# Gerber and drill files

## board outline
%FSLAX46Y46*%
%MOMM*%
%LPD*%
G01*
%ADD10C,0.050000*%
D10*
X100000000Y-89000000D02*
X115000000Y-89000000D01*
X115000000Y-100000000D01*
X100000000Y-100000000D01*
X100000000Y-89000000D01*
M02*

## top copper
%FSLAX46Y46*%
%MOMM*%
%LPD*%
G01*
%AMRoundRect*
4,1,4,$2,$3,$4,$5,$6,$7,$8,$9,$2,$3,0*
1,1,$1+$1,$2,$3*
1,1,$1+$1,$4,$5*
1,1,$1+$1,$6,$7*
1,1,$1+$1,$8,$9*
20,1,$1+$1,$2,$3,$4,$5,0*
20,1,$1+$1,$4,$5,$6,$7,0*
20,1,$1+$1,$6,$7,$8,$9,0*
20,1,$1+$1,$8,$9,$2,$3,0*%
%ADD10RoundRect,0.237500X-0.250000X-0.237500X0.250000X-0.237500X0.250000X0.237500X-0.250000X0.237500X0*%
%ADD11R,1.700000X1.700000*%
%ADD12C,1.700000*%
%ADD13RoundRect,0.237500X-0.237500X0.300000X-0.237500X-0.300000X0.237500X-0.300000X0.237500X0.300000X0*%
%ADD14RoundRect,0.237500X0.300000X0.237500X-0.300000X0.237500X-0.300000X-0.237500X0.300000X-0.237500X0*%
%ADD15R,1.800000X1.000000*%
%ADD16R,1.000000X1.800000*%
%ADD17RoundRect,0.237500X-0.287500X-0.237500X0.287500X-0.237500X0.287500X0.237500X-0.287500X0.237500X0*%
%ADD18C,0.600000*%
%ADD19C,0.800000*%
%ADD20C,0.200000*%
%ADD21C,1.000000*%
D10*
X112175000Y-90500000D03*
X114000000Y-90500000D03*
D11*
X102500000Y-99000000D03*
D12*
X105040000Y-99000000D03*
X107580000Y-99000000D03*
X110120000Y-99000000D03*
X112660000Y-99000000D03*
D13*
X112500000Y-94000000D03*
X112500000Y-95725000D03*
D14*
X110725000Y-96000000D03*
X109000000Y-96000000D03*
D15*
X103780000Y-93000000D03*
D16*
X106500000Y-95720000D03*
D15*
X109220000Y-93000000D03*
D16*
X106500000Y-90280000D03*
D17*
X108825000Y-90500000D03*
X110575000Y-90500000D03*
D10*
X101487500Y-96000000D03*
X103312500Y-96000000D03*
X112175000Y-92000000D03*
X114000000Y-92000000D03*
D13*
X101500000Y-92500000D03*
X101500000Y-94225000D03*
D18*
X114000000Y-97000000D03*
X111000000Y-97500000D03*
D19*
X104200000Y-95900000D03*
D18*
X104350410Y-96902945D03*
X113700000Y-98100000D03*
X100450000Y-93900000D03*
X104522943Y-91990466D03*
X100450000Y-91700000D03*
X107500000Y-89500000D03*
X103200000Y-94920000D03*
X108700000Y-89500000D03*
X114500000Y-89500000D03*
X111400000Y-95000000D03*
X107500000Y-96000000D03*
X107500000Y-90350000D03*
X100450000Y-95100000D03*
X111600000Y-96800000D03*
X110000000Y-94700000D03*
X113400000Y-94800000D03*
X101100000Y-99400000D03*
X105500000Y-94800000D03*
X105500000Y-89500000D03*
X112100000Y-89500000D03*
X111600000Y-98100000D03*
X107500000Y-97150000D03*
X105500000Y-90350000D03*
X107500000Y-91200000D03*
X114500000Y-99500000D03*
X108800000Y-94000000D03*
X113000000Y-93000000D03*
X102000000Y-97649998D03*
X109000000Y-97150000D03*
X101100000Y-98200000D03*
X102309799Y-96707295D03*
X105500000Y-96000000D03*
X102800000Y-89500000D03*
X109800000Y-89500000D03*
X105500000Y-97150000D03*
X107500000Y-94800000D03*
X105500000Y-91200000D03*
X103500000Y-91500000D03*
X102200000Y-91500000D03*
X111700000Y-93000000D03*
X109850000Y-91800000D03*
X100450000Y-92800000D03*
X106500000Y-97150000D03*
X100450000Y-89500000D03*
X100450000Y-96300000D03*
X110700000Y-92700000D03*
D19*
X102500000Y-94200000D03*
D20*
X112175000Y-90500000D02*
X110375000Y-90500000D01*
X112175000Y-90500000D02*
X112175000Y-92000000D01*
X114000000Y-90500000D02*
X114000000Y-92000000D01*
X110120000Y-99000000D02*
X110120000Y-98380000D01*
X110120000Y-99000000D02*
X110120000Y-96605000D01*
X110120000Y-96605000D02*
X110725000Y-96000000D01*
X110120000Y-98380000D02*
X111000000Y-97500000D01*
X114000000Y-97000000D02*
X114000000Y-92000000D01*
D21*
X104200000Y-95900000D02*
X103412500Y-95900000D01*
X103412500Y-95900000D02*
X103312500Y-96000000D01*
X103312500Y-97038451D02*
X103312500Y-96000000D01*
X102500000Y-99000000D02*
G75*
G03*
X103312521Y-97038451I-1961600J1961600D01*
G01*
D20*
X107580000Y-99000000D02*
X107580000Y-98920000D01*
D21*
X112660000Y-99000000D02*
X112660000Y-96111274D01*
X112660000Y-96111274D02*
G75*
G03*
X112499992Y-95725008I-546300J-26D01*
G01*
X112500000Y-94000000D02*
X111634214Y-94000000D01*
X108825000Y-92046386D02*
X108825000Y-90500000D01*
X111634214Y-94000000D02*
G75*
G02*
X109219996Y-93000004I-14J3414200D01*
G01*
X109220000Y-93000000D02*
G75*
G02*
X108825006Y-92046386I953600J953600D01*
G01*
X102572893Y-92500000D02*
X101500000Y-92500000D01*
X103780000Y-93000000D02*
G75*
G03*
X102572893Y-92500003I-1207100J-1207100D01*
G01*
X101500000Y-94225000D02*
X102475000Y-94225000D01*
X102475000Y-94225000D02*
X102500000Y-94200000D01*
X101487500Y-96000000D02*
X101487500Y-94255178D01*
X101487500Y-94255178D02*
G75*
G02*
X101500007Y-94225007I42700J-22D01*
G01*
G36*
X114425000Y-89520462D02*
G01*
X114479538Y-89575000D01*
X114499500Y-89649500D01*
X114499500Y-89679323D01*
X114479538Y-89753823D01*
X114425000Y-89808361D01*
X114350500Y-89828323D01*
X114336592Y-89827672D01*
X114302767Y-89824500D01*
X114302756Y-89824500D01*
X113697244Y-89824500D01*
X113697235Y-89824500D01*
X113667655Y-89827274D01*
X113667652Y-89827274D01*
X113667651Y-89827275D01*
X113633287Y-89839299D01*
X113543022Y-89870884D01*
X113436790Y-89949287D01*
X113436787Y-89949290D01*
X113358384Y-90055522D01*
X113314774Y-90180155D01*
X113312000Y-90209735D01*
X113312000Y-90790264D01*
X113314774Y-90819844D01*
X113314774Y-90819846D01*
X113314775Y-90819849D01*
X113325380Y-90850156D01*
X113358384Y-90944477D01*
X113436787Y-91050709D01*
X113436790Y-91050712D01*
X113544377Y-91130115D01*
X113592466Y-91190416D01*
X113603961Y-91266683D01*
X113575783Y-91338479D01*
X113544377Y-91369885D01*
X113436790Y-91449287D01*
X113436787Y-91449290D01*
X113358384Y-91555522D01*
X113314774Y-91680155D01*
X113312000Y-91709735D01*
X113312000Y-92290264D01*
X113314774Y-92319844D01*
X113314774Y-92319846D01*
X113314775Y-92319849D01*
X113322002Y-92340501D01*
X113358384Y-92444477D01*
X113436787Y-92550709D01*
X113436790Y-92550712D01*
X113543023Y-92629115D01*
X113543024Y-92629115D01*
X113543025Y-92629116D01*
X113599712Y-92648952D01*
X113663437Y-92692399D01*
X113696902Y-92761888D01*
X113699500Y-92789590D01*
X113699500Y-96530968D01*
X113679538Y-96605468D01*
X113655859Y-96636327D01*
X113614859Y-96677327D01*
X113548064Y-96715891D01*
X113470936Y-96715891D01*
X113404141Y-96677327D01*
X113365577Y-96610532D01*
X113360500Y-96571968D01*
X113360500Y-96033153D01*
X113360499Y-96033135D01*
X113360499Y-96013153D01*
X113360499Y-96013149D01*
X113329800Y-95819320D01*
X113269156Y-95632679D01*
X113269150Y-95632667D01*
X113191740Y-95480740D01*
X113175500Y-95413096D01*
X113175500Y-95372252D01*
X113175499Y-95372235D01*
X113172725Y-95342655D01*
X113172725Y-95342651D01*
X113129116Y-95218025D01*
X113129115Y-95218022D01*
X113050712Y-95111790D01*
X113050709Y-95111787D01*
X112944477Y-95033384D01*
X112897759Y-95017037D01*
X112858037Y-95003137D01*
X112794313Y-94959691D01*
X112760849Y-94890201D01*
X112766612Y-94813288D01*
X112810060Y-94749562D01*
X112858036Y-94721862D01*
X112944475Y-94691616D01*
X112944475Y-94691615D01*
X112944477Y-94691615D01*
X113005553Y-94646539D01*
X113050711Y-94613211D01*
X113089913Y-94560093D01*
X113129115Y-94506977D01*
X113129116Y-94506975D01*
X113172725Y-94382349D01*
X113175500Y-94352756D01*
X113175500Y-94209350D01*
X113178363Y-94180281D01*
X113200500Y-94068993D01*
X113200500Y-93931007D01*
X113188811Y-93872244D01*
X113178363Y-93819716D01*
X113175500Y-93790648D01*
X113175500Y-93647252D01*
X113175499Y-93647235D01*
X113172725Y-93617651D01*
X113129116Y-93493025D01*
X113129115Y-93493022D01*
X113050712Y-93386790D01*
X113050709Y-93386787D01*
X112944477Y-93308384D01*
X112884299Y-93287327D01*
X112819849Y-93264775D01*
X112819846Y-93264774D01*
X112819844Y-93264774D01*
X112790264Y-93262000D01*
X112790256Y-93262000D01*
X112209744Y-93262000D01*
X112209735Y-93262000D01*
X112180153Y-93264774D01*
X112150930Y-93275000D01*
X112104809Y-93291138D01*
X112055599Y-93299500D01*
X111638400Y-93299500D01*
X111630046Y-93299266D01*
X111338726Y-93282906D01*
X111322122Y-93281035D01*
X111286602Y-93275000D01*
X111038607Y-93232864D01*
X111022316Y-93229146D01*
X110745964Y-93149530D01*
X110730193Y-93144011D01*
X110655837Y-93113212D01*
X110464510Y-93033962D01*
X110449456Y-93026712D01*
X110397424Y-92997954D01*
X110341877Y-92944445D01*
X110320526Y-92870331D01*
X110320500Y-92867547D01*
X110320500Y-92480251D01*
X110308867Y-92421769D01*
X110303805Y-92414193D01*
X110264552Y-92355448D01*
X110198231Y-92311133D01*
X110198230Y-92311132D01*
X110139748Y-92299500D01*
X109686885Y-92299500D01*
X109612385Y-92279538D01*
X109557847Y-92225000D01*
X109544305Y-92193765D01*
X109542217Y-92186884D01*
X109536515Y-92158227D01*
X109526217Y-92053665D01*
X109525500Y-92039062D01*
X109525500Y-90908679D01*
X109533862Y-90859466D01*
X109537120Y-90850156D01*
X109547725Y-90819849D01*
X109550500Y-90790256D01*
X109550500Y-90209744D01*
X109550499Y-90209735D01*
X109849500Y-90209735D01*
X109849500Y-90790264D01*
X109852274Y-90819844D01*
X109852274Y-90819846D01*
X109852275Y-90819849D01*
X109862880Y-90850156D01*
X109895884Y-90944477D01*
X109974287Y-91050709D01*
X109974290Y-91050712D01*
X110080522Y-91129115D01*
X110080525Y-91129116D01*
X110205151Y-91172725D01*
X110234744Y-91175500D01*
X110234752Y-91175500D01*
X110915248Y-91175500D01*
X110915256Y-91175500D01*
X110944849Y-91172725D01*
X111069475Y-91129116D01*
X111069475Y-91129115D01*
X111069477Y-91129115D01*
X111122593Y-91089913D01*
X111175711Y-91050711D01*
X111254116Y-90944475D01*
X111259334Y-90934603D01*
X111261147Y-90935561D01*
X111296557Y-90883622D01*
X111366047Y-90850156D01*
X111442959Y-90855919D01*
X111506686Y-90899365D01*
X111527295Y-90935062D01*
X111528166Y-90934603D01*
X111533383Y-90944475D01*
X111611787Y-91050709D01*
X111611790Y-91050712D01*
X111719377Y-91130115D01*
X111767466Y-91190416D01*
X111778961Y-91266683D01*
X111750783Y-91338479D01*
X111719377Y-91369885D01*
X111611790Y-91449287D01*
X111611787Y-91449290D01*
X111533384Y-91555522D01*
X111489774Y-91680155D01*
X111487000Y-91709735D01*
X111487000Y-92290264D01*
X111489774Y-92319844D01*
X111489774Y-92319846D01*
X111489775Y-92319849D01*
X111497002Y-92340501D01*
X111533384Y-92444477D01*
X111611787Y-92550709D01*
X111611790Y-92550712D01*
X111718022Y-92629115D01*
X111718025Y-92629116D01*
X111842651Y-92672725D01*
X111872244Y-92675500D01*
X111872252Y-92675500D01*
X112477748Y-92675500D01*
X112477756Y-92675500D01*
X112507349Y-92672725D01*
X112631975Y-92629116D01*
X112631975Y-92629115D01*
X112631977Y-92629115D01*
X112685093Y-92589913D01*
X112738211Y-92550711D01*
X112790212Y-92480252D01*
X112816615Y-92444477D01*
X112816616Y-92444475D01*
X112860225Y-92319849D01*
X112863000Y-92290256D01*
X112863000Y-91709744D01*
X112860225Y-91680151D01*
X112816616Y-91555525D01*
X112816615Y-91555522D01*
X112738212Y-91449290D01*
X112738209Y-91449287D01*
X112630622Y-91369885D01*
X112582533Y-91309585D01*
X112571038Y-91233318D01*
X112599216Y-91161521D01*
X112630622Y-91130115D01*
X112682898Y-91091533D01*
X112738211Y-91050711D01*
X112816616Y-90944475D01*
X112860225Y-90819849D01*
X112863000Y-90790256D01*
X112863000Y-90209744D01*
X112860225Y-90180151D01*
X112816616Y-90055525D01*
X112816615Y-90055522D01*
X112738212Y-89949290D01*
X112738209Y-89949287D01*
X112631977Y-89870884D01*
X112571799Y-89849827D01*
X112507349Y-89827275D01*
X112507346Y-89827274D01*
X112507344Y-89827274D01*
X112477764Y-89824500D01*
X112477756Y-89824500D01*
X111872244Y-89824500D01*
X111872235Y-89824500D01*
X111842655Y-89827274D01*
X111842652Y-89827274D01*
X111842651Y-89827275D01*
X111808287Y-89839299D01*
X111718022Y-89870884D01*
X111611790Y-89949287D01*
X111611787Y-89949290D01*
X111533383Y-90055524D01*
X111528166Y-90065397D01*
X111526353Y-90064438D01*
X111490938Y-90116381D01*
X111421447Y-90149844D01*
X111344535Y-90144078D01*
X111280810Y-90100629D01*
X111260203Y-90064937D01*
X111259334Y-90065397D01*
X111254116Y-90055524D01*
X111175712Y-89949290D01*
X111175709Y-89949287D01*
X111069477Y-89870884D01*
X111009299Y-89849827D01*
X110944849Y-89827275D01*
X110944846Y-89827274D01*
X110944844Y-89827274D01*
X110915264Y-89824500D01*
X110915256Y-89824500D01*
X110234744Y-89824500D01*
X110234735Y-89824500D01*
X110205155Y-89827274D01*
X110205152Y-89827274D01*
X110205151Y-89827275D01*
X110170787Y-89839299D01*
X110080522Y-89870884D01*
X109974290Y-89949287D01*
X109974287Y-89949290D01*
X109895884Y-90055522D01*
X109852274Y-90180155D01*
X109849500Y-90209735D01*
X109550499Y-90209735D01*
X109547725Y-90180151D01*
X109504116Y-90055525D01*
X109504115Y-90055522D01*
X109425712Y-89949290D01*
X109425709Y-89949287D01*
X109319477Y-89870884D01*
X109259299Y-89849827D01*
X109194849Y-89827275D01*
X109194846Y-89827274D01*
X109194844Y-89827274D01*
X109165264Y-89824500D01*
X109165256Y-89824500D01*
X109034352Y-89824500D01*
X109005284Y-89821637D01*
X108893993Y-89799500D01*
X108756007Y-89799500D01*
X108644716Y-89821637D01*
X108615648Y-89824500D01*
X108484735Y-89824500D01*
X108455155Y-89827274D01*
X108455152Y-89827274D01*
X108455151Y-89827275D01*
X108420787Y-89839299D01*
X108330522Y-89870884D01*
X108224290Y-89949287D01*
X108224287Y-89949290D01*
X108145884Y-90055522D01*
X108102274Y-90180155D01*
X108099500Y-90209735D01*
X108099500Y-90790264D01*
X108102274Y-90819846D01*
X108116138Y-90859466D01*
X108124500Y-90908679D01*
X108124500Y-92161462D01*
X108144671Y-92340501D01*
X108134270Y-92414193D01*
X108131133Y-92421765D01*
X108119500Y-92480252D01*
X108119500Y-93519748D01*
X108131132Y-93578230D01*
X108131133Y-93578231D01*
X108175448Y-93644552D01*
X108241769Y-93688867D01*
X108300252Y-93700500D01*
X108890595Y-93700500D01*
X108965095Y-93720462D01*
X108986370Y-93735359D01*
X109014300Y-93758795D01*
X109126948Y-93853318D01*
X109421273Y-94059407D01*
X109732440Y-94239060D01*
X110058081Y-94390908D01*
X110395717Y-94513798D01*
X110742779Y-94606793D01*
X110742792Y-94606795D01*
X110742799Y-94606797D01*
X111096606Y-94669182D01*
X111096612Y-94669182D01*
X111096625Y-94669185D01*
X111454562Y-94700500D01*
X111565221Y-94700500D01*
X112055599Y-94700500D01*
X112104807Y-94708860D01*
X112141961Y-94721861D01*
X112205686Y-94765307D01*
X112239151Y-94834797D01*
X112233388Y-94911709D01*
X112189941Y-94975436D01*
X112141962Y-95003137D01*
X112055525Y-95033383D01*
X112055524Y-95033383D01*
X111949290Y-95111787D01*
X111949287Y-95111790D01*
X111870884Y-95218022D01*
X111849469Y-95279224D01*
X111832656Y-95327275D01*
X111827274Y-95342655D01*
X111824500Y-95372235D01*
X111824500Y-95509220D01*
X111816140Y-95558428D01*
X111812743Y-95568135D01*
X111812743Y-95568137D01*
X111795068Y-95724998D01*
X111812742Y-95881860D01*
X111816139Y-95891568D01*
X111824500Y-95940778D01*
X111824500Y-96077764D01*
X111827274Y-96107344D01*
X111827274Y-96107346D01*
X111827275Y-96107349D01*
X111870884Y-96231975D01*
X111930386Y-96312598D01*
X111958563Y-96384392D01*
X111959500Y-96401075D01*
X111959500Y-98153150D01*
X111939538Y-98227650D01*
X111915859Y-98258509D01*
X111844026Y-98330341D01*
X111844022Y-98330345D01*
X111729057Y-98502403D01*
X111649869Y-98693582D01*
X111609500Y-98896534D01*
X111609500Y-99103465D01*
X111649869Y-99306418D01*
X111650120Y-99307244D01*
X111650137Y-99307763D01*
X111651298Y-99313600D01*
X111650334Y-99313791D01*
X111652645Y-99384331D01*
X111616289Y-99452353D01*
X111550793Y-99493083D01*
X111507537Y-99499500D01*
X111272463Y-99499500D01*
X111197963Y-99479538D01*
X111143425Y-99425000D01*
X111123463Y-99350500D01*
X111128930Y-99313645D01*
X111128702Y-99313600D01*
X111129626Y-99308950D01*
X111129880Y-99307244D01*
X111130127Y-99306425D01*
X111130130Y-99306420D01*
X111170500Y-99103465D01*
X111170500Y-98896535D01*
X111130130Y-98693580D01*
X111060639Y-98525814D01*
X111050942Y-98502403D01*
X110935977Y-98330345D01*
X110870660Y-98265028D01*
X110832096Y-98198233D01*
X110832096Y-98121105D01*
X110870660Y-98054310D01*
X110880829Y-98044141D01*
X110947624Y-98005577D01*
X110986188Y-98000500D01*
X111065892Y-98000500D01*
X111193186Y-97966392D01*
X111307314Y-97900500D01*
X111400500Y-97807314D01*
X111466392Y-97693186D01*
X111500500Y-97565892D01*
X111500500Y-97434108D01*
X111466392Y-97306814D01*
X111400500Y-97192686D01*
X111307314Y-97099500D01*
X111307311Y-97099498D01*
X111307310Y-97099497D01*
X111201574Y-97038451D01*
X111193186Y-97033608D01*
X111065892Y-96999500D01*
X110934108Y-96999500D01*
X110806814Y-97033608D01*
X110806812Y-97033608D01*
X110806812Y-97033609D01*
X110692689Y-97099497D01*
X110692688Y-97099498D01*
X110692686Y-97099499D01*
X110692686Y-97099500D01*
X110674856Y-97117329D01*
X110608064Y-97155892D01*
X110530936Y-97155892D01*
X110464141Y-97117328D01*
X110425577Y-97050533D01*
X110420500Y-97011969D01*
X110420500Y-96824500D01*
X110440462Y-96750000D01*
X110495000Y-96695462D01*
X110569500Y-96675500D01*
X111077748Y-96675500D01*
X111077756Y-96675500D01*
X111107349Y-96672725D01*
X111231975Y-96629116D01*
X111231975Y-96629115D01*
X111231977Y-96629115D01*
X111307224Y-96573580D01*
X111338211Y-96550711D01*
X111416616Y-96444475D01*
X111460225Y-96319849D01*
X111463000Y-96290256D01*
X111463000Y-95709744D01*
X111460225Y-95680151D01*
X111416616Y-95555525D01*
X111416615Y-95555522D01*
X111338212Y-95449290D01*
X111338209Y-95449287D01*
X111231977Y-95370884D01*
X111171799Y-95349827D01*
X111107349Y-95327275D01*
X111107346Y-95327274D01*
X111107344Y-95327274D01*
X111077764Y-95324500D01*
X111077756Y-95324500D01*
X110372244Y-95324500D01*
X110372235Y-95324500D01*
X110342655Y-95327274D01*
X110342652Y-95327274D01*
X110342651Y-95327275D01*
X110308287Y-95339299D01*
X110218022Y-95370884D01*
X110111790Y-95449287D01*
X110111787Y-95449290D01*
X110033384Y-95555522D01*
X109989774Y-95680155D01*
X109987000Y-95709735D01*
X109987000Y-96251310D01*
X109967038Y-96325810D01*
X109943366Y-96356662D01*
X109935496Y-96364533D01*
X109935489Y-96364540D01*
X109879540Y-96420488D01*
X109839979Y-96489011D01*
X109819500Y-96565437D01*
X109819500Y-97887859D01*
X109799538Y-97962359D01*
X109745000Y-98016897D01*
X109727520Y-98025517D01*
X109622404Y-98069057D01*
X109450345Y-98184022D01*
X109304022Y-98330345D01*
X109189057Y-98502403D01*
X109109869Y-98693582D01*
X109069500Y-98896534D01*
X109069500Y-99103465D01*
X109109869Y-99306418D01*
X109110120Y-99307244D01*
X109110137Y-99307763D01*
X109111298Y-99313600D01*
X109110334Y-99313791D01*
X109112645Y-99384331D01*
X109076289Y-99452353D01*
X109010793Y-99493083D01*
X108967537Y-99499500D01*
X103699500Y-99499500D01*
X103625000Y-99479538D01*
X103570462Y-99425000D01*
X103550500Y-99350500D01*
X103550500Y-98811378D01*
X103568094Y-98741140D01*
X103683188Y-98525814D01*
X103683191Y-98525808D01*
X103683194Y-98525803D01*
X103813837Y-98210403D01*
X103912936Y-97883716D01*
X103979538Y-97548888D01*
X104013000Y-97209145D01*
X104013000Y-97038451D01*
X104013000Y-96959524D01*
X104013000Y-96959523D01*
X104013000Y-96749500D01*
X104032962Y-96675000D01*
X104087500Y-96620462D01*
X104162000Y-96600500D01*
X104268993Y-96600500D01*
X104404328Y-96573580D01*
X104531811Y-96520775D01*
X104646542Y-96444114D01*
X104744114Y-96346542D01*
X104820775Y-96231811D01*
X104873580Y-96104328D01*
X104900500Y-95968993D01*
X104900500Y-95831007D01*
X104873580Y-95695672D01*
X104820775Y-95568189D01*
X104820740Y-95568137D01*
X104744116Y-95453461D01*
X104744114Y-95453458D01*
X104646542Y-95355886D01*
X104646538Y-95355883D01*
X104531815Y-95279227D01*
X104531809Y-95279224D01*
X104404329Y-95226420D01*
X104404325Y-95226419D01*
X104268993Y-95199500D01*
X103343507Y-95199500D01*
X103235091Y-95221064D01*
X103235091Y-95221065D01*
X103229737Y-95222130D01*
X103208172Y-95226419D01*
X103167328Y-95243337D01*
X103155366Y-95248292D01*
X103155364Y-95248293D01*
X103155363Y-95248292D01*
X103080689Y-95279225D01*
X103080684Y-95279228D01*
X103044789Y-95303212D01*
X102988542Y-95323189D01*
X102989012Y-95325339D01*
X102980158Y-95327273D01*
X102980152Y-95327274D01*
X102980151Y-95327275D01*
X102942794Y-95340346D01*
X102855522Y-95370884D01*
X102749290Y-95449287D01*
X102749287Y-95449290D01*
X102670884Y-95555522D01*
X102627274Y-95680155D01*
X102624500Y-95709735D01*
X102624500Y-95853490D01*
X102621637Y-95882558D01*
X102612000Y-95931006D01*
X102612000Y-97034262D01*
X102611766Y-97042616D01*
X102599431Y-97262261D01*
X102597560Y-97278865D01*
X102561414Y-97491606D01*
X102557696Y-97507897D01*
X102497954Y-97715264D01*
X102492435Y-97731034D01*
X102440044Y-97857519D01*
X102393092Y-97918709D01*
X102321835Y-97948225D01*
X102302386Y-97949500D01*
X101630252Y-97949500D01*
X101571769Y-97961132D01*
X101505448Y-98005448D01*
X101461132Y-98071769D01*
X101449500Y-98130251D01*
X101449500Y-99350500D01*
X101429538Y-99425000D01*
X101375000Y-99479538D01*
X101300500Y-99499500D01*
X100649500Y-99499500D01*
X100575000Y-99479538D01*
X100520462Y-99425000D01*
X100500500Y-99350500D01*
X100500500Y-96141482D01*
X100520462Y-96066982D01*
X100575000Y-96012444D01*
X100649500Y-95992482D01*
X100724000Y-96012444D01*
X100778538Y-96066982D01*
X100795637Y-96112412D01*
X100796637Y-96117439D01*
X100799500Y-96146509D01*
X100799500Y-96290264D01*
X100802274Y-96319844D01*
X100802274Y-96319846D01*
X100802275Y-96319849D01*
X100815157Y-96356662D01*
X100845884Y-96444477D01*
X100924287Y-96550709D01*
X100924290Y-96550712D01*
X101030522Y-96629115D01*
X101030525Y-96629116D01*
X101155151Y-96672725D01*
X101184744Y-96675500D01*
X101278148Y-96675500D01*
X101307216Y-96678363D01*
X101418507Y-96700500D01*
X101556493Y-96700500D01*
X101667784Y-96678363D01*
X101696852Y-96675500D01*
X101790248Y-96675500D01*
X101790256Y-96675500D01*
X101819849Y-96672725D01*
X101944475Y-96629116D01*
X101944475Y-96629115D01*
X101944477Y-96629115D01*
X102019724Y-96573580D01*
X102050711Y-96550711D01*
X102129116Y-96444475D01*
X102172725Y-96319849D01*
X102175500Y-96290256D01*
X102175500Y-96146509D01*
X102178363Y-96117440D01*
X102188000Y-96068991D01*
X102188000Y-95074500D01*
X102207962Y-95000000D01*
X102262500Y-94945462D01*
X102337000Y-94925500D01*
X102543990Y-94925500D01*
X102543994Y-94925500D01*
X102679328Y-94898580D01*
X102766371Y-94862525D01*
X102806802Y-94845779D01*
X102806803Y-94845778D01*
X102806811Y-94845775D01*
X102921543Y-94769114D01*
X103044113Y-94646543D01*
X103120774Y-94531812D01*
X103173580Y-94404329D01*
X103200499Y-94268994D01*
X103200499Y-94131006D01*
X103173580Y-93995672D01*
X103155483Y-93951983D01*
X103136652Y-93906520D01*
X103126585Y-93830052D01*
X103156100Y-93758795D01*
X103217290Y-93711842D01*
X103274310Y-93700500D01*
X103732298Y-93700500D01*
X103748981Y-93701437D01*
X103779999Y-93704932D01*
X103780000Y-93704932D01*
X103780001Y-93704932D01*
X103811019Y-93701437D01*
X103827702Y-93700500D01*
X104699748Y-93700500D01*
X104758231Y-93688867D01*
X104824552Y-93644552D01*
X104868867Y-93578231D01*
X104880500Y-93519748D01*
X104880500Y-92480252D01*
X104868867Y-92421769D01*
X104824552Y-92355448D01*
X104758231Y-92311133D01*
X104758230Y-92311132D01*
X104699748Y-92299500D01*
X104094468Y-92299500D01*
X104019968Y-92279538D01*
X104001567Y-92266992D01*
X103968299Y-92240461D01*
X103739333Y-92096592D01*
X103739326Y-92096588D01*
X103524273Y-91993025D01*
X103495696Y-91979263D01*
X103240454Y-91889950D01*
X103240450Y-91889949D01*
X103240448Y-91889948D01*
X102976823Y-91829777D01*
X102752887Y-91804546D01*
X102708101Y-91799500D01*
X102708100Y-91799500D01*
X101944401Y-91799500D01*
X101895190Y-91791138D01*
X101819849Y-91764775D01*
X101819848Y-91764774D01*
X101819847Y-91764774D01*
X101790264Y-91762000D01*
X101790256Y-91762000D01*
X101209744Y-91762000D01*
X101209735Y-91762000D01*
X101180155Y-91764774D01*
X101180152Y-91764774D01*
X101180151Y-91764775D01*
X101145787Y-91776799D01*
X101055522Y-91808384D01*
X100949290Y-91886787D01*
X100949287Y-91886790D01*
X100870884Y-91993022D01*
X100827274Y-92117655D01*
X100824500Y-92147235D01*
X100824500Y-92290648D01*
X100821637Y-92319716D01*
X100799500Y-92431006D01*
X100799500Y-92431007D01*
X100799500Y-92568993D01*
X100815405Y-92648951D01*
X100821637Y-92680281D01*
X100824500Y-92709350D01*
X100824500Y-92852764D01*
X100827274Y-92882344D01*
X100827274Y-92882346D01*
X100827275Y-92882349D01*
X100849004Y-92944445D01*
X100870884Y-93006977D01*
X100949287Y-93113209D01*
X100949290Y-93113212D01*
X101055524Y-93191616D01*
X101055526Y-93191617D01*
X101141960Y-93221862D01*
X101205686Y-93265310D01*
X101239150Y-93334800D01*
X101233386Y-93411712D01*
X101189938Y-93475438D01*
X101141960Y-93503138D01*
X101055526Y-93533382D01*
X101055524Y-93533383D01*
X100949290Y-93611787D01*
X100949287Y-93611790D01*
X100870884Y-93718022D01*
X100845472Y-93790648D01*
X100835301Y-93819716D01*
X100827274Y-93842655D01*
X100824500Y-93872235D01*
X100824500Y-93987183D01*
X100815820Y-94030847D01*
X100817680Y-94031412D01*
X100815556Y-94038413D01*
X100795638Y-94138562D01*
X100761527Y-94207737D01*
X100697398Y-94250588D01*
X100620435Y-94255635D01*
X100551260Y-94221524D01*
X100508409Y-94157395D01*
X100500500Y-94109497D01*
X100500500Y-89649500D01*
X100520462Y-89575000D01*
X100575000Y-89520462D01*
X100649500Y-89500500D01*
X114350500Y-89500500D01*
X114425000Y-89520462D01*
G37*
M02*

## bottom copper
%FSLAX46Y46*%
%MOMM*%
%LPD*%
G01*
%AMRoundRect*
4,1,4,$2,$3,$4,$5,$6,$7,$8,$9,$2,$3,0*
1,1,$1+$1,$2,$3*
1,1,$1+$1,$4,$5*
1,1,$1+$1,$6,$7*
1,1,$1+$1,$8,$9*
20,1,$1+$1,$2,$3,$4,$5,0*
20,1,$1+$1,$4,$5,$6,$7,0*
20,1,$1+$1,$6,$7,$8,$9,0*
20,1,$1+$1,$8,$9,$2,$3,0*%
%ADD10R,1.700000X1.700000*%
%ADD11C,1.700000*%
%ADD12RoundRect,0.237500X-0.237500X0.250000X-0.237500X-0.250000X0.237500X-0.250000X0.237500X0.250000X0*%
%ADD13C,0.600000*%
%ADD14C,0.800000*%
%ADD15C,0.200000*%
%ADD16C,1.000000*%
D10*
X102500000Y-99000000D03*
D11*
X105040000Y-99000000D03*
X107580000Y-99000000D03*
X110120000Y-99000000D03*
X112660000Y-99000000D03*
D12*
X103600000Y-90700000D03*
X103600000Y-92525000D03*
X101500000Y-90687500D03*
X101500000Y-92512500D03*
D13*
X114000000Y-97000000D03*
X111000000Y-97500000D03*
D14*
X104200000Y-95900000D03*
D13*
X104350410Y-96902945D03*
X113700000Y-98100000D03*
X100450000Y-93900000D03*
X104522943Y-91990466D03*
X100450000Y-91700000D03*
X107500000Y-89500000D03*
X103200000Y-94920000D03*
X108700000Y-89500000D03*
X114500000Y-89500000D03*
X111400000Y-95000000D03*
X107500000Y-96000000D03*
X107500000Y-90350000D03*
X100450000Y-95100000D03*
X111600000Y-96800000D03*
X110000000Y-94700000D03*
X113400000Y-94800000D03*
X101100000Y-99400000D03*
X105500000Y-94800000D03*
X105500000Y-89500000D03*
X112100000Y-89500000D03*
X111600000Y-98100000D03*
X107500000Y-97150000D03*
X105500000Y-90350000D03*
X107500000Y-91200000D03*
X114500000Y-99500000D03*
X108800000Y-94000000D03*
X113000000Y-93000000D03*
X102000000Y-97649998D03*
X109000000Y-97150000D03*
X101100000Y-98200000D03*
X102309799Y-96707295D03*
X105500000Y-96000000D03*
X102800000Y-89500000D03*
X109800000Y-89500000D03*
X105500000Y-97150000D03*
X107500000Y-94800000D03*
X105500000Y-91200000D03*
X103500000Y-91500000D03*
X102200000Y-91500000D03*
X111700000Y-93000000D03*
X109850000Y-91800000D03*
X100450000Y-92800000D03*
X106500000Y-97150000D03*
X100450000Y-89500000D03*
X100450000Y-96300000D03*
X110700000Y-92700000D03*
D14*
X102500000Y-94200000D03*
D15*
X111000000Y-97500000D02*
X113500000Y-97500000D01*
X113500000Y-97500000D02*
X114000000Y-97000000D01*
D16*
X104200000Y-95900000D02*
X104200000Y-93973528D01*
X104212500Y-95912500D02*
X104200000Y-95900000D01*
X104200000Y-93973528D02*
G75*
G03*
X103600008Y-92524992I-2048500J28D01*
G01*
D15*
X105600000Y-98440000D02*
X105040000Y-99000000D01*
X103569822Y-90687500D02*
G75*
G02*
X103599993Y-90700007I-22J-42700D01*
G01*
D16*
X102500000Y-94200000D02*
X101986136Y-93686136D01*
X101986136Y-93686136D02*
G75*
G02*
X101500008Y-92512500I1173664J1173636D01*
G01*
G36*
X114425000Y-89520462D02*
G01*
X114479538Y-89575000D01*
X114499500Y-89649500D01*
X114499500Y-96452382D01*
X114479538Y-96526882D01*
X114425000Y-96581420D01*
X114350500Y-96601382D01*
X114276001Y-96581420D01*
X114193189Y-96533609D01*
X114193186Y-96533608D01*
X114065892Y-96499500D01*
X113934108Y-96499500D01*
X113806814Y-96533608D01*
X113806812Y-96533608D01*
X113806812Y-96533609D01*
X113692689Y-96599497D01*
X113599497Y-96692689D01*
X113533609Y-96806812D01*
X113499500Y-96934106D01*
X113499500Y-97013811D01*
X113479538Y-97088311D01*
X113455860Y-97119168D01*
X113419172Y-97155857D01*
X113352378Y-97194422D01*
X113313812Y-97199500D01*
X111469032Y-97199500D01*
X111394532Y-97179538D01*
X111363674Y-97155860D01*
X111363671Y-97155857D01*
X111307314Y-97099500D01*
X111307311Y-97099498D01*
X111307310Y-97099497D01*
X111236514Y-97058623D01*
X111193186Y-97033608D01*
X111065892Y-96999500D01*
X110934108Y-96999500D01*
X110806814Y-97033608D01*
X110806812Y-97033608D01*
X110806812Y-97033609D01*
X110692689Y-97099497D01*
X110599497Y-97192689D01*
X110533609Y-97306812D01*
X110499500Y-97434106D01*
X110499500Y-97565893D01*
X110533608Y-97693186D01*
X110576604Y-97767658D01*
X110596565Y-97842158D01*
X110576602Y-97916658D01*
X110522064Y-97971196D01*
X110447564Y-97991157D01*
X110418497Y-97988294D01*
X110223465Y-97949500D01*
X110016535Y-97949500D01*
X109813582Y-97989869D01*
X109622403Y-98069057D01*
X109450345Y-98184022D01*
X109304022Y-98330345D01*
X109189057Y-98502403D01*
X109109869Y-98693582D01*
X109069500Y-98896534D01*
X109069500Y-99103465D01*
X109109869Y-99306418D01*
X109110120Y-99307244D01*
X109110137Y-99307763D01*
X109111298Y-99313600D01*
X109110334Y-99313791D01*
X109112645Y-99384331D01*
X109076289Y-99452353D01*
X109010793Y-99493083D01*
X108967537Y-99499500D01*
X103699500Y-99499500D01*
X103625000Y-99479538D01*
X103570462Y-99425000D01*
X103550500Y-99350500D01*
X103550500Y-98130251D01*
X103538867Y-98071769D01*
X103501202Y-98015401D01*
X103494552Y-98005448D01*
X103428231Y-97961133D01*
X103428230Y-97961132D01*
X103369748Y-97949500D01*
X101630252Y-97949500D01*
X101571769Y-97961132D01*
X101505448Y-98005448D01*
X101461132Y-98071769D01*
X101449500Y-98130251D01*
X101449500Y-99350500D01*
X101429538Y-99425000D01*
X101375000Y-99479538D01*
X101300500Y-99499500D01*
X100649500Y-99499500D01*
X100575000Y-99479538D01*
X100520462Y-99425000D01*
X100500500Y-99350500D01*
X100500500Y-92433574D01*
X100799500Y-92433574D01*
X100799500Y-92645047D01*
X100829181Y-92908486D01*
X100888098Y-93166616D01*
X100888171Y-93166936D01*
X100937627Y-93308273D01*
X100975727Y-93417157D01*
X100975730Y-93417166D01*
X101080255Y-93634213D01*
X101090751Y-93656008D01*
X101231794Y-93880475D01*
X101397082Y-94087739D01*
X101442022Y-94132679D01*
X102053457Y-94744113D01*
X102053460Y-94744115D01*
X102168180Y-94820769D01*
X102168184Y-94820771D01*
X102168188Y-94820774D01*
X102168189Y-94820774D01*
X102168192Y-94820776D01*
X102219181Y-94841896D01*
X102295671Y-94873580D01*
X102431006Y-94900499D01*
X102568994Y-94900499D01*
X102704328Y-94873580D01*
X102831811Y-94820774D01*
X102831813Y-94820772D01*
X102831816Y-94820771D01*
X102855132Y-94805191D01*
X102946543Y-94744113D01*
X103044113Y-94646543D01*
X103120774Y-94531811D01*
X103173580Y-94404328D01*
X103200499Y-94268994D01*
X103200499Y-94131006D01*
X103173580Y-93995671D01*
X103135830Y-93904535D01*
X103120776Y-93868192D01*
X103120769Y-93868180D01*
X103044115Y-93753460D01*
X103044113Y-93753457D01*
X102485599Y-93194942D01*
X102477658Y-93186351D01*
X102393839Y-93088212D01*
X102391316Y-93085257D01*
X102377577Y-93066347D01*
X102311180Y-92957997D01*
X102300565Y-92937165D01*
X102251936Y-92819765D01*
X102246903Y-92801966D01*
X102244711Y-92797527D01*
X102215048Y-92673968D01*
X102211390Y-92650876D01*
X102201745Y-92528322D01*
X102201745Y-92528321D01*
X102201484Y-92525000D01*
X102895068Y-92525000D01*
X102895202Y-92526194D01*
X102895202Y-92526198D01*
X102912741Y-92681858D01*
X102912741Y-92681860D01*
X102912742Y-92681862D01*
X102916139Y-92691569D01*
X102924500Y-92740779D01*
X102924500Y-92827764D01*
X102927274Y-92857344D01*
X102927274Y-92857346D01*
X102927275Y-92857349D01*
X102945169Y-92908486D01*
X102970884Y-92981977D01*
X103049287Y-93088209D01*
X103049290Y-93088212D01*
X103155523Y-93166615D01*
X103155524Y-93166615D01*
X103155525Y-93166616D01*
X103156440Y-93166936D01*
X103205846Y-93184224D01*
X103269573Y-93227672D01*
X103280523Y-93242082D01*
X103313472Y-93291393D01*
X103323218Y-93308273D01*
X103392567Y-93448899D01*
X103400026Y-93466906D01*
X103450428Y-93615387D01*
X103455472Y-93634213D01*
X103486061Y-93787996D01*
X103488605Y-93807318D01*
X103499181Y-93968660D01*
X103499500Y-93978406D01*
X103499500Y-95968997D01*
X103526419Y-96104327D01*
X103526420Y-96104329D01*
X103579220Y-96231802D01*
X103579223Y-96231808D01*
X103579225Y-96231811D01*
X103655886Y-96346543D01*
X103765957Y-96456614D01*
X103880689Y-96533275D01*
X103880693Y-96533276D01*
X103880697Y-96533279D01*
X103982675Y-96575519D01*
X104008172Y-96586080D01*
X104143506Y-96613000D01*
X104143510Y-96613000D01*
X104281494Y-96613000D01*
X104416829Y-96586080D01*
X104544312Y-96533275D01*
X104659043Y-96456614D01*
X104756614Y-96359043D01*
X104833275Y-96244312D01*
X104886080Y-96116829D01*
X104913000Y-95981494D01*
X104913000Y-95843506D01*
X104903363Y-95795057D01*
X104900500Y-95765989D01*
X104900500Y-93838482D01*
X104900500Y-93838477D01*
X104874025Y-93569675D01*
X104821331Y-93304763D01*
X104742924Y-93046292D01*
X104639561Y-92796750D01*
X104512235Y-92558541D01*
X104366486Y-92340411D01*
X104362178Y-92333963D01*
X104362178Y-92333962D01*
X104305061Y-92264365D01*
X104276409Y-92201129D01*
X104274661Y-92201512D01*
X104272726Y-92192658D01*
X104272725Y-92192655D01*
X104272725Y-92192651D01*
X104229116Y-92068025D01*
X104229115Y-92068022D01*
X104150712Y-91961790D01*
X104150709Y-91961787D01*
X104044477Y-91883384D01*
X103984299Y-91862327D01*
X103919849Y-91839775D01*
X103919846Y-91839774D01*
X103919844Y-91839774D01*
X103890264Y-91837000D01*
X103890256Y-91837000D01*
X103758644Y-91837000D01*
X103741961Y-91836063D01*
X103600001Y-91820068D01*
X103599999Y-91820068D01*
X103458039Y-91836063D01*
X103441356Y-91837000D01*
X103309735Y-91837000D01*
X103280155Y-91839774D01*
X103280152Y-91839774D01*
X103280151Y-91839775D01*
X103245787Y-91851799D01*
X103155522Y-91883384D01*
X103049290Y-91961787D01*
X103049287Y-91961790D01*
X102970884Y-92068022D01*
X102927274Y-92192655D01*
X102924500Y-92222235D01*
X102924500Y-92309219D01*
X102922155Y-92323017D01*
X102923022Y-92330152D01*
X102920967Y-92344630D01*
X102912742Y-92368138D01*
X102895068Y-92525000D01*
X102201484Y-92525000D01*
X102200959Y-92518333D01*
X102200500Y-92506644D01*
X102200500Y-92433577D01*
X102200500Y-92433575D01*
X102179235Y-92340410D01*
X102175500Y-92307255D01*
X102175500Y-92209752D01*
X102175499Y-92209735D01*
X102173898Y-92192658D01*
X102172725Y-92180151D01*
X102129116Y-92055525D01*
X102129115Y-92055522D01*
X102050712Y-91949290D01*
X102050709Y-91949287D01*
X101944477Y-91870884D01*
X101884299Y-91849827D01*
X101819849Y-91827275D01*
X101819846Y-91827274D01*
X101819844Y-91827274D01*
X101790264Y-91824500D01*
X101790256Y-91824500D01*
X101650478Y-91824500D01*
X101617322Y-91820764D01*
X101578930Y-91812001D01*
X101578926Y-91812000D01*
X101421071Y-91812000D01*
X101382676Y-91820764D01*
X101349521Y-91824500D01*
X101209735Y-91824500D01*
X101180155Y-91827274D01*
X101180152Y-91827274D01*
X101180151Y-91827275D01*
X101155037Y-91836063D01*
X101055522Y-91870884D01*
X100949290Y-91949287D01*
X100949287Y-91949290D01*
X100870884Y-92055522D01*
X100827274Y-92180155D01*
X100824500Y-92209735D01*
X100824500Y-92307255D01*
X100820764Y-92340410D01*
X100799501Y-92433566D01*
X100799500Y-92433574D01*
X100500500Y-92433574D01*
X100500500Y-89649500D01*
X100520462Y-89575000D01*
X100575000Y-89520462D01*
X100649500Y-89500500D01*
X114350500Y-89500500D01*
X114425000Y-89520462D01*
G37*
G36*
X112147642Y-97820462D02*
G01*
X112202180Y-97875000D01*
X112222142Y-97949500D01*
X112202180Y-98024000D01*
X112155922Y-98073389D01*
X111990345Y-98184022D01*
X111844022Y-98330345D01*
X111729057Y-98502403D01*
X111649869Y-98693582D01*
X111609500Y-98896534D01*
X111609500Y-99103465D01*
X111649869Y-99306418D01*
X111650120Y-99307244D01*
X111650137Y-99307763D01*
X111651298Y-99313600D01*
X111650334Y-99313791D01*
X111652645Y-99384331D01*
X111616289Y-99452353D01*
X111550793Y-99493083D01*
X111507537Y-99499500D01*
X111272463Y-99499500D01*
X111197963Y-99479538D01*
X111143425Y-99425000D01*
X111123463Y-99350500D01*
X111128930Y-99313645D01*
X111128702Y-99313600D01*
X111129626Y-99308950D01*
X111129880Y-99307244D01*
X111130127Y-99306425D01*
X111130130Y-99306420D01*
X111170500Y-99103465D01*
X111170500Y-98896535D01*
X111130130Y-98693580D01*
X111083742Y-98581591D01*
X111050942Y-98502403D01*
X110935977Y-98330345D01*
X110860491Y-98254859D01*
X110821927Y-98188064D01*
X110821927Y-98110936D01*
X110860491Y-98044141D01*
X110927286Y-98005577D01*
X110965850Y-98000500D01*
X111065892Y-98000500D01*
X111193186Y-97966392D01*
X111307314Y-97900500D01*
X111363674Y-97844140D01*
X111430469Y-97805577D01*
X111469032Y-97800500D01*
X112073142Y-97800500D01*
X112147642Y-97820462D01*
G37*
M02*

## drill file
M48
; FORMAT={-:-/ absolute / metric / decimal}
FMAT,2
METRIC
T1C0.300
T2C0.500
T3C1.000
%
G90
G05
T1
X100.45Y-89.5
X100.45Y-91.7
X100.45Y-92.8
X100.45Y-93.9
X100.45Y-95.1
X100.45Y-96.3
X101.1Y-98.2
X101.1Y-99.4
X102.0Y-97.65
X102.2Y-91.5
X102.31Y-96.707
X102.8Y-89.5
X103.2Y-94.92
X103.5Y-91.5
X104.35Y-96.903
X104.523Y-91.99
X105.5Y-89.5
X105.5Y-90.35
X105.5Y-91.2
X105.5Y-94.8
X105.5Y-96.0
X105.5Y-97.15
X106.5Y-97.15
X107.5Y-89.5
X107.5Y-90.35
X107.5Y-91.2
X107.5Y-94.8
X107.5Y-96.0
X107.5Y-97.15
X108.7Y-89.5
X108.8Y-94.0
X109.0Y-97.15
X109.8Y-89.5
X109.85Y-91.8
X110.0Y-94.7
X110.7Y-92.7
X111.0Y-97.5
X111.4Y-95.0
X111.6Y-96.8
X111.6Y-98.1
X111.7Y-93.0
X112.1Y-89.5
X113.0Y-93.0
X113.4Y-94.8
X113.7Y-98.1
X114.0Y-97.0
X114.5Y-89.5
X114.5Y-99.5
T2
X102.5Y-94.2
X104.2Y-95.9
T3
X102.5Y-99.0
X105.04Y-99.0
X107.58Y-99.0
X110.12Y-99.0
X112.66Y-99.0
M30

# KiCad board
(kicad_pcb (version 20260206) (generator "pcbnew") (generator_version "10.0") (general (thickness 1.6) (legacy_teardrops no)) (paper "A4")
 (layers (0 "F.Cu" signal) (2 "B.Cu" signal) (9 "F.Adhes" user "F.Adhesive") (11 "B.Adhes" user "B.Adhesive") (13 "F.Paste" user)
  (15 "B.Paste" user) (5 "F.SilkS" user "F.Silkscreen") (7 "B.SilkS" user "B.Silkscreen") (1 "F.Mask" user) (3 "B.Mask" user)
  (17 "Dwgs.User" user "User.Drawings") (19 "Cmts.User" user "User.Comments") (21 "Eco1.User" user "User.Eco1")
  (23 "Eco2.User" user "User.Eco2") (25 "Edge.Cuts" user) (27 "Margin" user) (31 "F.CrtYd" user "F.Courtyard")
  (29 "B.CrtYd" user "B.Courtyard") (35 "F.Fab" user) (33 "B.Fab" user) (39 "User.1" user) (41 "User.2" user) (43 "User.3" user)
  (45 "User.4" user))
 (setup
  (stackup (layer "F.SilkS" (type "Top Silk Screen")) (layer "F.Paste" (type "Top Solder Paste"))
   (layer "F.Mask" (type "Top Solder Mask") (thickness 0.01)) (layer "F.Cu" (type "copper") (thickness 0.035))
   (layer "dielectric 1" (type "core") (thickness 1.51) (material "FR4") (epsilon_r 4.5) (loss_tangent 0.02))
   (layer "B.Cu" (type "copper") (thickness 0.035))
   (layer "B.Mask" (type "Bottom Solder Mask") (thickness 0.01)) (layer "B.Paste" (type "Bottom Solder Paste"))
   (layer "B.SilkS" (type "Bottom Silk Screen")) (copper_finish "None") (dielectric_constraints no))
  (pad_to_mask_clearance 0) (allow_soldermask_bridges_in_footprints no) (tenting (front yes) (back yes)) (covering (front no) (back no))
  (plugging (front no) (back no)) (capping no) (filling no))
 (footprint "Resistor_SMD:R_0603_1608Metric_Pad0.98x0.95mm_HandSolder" (layer "F.Cu") (at 113.0875 90.5)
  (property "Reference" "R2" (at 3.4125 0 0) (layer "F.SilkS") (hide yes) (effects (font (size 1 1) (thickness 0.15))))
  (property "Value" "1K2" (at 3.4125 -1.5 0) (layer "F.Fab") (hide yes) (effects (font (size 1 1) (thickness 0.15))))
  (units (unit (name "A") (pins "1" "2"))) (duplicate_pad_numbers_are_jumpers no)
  (pad "1" smd roundrect (at -0.9125 0) (size 0.975 0.95) (layers "F.Cu" "F.Mask" "F.Paste") (roundrect_rratio 0.25) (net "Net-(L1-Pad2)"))
  (pad "2" smd roundrect (at 0.9125 0) (size 0.975 0.95) (layers "F.Cu" "F.Mask" "F.Paste") (roundrect_rratio 0.25) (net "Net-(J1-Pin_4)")))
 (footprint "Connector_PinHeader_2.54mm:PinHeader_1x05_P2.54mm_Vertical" (layer "F.Cu") (at 102.5 99 90)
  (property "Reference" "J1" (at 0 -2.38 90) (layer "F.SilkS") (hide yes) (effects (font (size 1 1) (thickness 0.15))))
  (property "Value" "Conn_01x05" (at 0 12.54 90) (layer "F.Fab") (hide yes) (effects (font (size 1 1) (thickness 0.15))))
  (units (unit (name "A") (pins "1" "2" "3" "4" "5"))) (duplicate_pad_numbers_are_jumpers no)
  (pad "1" thru_hole rect (at 0 0 90) (size 1.7 1.7) (drill 1) (layers "*.Cu" "*.Mask") (remove_unused_layers no) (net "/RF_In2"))
  (pad "2" thru_hole circle (at 0 2.54 90) (size 1.7 1.7) (drill 1) (layers "*.Cu" "*.Mask") (remove_unused_layers no) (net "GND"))
  (pad "3" thru_hole circle (at 0 5.08 90) (size 1.7 1.7) (drill 1) (layers "*.Cu" "*.Mask") (remove_unused_layers no) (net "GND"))
  (pad "4" thru_hole circle (at 0 7.62 90) (size 1.7 1.7) (drill 1) (layers "*.Cu" "*.Mask") (remove_unused_layers no)
   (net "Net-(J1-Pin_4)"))
  (pad "5" thru_hole circle (at 0 10.16 90) (size 1.7 1.7) (drill 1) (layers "*.Cu" "*.Mask") (remove_unused_layers no) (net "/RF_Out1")))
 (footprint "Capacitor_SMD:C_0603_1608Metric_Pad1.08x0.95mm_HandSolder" (layer "F.Cu") (at 112.5 94.8625 -90)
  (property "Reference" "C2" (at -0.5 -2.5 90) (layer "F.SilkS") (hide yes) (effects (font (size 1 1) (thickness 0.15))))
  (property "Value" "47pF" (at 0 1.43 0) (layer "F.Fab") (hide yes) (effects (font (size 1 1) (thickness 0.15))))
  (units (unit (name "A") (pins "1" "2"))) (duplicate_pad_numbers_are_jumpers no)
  (pad "1" smd roundrect (at -0.8625 0 270) (size 1.075 0.95) (layers "F.Cu" "F.Mask" "F.Paste") (roundrect_rratio 0.25) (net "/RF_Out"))
  (pad "2" smd roundrect (at 0.8625 0 270) (size 1.075 0.95) (layers "F.Cu" "F.Mask" "F.Paste") (roundrect_rratio 0.25) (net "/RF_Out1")))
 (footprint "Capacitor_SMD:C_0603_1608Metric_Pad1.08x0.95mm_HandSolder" (layer "F.Cu") (at 109.8625 96 180)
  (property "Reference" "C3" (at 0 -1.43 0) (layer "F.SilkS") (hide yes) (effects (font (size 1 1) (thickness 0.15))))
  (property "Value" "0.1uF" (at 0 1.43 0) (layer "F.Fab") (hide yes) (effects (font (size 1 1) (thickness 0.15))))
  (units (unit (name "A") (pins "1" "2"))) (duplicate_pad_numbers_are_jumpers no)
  (pad "1" smd roundrect (at -0.8625 0 180) (size 1.075 0.95) (layers "F.Cu" "F.Mask" "F.Paste") (roundrect_rratio 0.25)
   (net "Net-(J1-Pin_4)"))
  (pad "2" smd roundrect (at 0.8625 0 180) (size 1.075 0.95) (layers "F.Cu" "F.Mask" "F.Paste") (roundrect_rratio 0.25) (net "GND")))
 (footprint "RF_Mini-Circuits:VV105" (layer "F.Cu") (at 106.5 93 -90)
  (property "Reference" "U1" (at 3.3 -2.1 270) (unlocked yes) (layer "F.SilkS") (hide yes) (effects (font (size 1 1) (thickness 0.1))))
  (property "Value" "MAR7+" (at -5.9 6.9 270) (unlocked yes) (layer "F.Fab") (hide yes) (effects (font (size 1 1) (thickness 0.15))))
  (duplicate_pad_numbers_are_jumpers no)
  (pad "1" smd rect (at 0 2.72 180) (size 1.8 1) (layers "F.Cu" "F.Mask") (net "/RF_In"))
  (pad "2" smd rect (at 2.72 0 270) (size 1.8 1) (layers "F.Cu" "F.Mask") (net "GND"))
  (pad "3" smd rect (at 0 -2.72 180) (size 1.8 1) (layers "F.Cu" "F.Mask") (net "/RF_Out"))
  (pad "4" smd rect (at -2.72 0 270) (size 1.8 1) (layers "F.Cu" "F.Mask") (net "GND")))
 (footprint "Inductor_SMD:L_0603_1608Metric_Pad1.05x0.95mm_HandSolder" (layer "F.Cu") (at 109.7 90.5)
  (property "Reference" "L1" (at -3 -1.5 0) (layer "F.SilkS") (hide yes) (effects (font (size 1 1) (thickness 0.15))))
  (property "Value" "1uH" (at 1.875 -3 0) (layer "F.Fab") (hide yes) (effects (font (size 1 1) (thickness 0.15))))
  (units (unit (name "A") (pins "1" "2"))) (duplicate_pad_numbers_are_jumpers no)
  (pad "1" smd roundrect (at -0.875 0) (size 1.05 0.95) (layers "F.Cu" "F.Mask" "F.Paste") (roundrect_rratio 0.25) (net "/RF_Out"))
  (pad "2" smd roundrect (at 0.875 0) (size 1.05 0.95) (layers "F.Cu" "F.Mask" "F.Paste") (roundrect_rratio 0.25) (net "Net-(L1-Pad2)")))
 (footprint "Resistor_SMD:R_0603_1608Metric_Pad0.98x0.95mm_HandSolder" (layer "F.Cu") (at 102.4 96)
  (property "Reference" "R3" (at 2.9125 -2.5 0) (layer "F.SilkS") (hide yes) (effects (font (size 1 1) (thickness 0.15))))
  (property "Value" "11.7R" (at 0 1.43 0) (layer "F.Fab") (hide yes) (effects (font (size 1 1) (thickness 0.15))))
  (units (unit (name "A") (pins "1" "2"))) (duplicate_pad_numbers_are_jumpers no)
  (pad "1" smd roundrect (at -0.9125 0) (size 0.975 0.95) (layers "F.Cu" "F.Mask" "F.Paste") (roundrect_rratio 0.25) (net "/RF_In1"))
  (pad "2" smd roundrect (at 0.9125 0) (size 0.975 0.95) (layers "F.Cu" "F.Mask" "F.Paste") (roundrect_rratio 0.25) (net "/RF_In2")))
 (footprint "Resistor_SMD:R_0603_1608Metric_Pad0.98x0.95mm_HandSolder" (layer "F.Cu") (at 113.0875 92)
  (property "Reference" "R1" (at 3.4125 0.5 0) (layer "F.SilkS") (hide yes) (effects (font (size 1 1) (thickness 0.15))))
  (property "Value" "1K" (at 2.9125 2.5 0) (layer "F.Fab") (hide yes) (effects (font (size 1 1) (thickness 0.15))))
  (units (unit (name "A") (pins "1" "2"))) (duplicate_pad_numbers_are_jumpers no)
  (pad "1" smd roundrect (at -0.9125 0) (size 0.975 0.95) (layers "F.Cu" "F.Mask" "F.Paste") (roundrect_rratio 0.25) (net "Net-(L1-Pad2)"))
  (pad "2" smd roundrect (at 0.9125 0) (size 0.975 0.95) (layers "F.Cu" "F.Mask" "F.Paste") (roundrect_rratio 0.25) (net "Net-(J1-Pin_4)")))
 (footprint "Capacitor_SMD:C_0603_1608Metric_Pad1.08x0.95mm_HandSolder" (layer "F.Cu") (at 101.5 93.3625 -90)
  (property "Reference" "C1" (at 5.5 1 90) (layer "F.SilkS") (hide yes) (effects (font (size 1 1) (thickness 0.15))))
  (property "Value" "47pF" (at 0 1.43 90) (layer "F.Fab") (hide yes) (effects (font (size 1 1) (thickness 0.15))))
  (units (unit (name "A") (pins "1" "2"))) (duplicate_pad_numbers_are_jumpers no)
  (pad "1" smd roundrect (at -0.8625 0 270) (size 1.075 0.95) (layers "F.Cu" "F.Mask" "F.Paste") (roundrect_rratio 0.25) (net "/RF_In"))
  (pad "2" smd roundrect (at 0.8625 0 270) (size 1.075 0.95) (layers "F.Cu" "F.Mask" "F.Paste") (roundrect_rratio 0.25) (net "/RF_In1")))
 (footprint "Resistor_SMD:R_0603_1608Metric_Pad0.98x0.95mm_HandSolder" (layer "B.Cu") (at 103.6 91.6125 -90)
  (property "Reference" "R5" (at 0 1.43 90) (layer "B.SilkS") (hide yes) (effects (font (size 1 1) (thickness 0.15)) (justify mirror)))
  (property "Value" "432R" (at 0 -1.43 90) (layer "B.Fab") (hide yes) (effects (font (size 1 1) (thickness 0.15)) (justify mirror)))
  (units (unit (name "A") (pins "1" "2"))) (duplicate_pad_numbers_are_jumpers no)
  (pad "1" smd roundrect (at -0.9125 0 270) (size 0.975 0.95) (layers "B.Cu" "B.Mask" "B.Paste") (roundrect_rratio 0.25) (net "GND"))
  (pad "2" smd roundrect (at 0.9125 0 270) (size 0.975 0.95) (layers "B.Cu" "B.Mask" "B.Paste") (roundrect_rratio 0.25) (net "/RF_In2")))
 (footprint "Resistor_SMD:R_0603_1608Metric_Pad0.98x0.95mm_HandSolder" (layer "B.Cu") (at 101.5 91.6 -90)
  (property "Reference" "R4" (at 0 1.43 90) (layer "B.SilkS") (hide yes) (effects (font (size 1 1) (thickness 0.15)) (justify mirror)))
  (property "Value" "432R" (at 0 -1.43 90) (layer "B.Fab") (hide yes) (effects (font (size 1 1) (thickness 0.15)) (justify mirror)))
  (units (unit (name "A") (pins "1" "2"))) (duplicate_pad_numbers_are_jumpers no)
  (pad "1" smd roundrect (at -0.9125 0 270) (size 0.975 0.95) (layers "B.Cu" "B.Mask" "B.Paste") (roundrect_rratio 0.25) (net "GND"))
  (pad "2" smd roundrect (at 0.9125 0 270) (size 0.975 0.95) (layers "B.Cu" "B.Mask" "B.Paste") (roundrect_rratio 0.25) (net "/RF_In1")))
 (gr_rect (start 100 89) (end 115 100) (stroke (width 0.05) (type default)) (fill no) (layer "Edge.Cuts"))
 (segment (start 112.175 90.5) (end 110.375 90.5) (width 0.2) (layer "F.Cu") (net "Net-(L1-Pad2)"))
 (segment (start 112.175 90.5) (end 112.175 92) (width 0.2) (layer "F.Cu") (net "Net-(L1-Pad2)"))
 (segment (start 114 90.5) (end 114 92) (width 0.2) (layer "F.Cu") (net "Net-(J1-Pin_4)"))
 (segment (start 110.12 99) (end 110.12 98.38) (width 0.2) (layer "F.Cu") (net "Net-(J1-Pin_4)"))
 (segment (start 110.12 99) (end 110.12 96.605) (width 0.2) (layer "F.Cu") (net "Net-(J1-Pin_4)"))
 (segment (start 110.12 96.605) (end 110.725 96) (width 0.2) (layer "F.Cu") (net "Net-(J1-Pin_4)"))
 (segment (start 110.12 98.38) (end 111 97.5) (width 0.2) (layer "F.Cu") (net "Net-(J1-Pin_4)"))
 (segment (start 114 97) (end 114 92) (width 0.2) (layer "F.Cu") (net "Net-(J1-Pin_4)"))
 (via (at 114 97) (size 0.6) (drill 0.3) (layers "F.Cu" "B.Cu") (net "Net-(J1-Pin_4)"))
 (via (at 111 97.5) (size 0.6) (drill 0.3) (layers "F.Cu" "B.Cu") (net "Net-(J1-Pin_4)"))
 (segment (start 111 97.5) (end 113.5 97.5) (width 0.2) (layer "B.Cu") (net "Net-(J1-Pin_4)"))
 (segment (start 113.5 97.5) (end 114 97) (width 0.2) (layer "B.Cu") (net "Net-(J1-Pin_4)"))
 (segment (start 104.2 95.9) (end 103.4125 95.9) (width 1) (layer "F.Cu") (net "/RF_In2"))
 (segment (start 103.4125 95.9) (end 103.3125 96) (width 1) (layer "F.Cu") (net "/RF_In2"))
 (segment (start 103.3125 97.038451) (end 103.3125 96) (width 1) (layer "F.Cu") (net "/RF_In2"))
 (via (at 104.2 95.9) (size 0.8) (drill 0.5) (layers "F.Cu" "B.Cu") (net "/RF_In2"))
 (arc (start 102.5 99) (mid 103.101338 98.100033) (end 103.3125 97.038451) (width 1) (layer "F.Cu") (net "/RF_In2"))
 (segment (start 104.2 95.9) (end 104.2 93.973528) (width 1) (layer "B.Cu") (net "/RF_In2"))
 (segment (start 104.2125 95.9125) (end 104.2 95.9) (width 1) (layer "B.Cu") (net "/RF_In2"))
 (arc (start 104.2 93.973528) (mid 104.044065 93.18959) (end 103.6 92.525) (width 1) (layer "B.Cu") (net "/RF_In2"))
 (segment (start 107.58 99) (end 107.58 98.92) (width 0.2) (layer "F.Cu") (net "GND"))
 (via (at 104.35041 96.902945) (size 0.6) (drill 0.3) (layers "F.Cu" "B.Cu") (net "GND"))
 (via (at 113.7 98.1) (size 0.6) (drill 0.3) (layers "F.Cu" "B.Cu") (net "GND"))
 (via (at 100.45 93.9) (size 0.6) (drill 0.3) (layers "F.Cu" "B.Cu") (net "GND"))
 (via (at 104.522943 91.990466) (size 0.6) (drill 0.3) (layers "F.Cu" "B.Cu") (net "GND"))
 (via (at 100.45 91.7) (size 0.6) (drill 0.3) (layers "F.Cu" "B.Cu") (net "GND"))
 (via (at 107.5 89.5) (size 0.6) (drill 0.3) (layers "F.Cu" "B.Cu") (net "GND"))
 (via (at 103.2 94.92) (size 0.6) (drill 0.3) (layers "F.Cu" "B.Cu") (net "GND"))
 (via (at 108.7 89.5) (size 0.6) (drill 0.3) (layers "F.Cu" "B.Cu") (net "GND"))
 (via (at 114.5 89.5) (size 0.6) (drill 0.3) (layers "F.Cu" "B.Cu") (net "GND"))
 (via (at 111.4 95) (size 0.6) (drill 0.3) (layers "F.Cu" "B.Cu") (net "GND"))
 (via (at 107.5 96) (size 0.6) (drill 0.3) (layers "F.Cu" "B.Cu") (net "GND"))
 (via (at 107.5 90.35) (size 0.6) (drill 0.3) (layers "F.Cu" "B.Cu") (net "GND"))
 (via (at 100.45 95.1) (size 0.6) (drill 0.3) (layers "F.Cu" "B.Cu") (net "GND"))
 (via (at 111.6 96.8) (size 0.6) (drill 0.3) (layers "F.Cu" "B.Cu") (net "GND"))
 (via (at 110 94.7) (size 0.6) (drill 0.3) (layers "F.Cu" "B.Cu") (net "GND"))
 (via (at 113.4 94.8) (size 0.6) (drill 0.3) (layers "F.Cu" "B.Cu") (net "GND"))
 (via (at 101.1 99.4) (size 0.6) (drill 0.3) (layers "F.Cu" "B.Cu") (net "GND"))
 (via (at 105.5 94.8) (size 0.6) (drill 0.3) (layers "F.Cu" "B.Cu") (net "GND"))
 (via (at 105.5 89.5) (size 0.6) (drill 0.3) (layers "F.Cu" "B.Cu") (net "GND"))
 (via (at 112.1 89.5) (size 0.6) (drill 0.3) (layers "F.Cu" "B.Cu") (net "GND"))
 (via (at 111.6 98.1) (size 0.6) (drill 0.3) (layers "F.Cu" "B.Cu") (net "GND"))
 (via (at 107.5 97.15) (size 0.6) (drill 0.3) (layers "F.Cu" "B.Cu") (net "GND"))
 (via (at 105.5 90.35) (size 0.6) (drill 0.3) (layers "F.Cu" "B.Cu") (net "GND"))
 (via (at 107.5 91.2) (size 0.6) (drill 0.3) (layers "F.Cu" "B.Cu") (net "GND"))
 (via (at 114.5 99.5) (size 0.6) (drill 0.3) (layers "F.Cu" "B.Cu") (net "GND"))
 (via (at 108.8 94) (size 0.6) (drill 0.3) (layers "F.Cu" "B.Cu") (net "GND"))
 (via (at 113 93) (size 0.6) (drill 0.3) (layers "F.Cu" "B.Cu") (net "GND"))
 (via (at 102 97.649998) (size 0.6) (drill 0.3) (layers "F.Cu" "B.Cu") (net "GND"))
 (via (at 109 97.15) (size 0.6) (drill 0.3) (layers "F.Cu" "B.Cu") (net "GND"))
 (via (at 101.1 98.2) (size 0.6) (drill 0.3) (layers "F.Cu" "B.Cu") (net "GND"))
 (via (at 102.309799 96.707295) (size 0.6) (drill 0.3) (layers "F.Cu" "B.Cu") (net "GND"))
 (via (at 105.5 96) (size 0.6) (drill 0.3) (layers "F.Cu" "B.Cu") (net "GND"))
 (via (at 102.8 89.5) (size 0.6) (drill 0.3) (layers "F.Cu" "B.Cu") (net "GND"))
 (via (at 109.8 89.5) (size 0.6) (drill 0.3) (layers "F.Cu" "B.Cu") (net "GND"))
 (via (at 105.5 97.15) (size 0.6) (drill 0.3) (layers "F.Cu" "B.Cu") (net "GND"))
 (via (at 107.5 94.8) (size 0.6) (drill 0.3) (layers "F.Cu" "B.Cu") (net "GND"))
 (via (at 105.5 91.2) (size 0.6) (drill 0.3) (layers "F.Cu" "B.Cu") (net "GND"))
 (via (at 103.5 91.5) (size 0.6) (drill 0.3) (layers "F.Cu" "B.Cu") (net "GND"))
 (via (at 102.2 91.5) (size 0.6) (drill 0.3) (layers "F.Cu" "B.Cu") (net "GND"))
 (via (at 111.7 93) (size 0.6) (drill 0.3) (layers "F.Cu" "B.Cu") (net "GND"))
 (via (at 109.85 91.8) (size 0.6) (drill 0.3) (layers "F.Cu" "B.Cu") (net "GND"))
 (via (at 100.45 92.8) (size 0.6) (drill 0.3) (layers "F.Cu" "B.Cu") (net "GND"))
 (via (at 106.5 97.15) (size 0.6) (drill 0.3) (layers "F.Cu" "B.Cu") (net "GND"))
 (via (at 100.45 89.5) (size 0.6) (drill 0.3) (layers "F.Cu" "B.Cu") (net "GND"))
 (via (at 100.45 96.3) (size 0.6) (drill 0.3) (layers "F.Cu" "B.Cu") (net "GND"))
 (via (at 110.7 92.7) (size 0.6) (drill 0.3) (layers "F.Cu" "B.Cu") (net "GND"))
 (segment (start 105.6 98.44) (end 105.04 99) (width 0.2) (layer "B.Cu") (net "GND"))
 (arc (start 103.569822 90.6875) (mid 103.586154 90.690749) (end 103.6 90.7) (width 0.2) (layer "B.Cu") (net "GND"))
 (segment (start 112.66 99) (end 112.66 96.111274) (width 1) (layer "F.Cu") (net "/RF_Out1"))
 (arc (start 112.66 96.111274) (mid 112.618417 95.902224) (end 112.5 95.725) (width 1) (layer "F.Cu") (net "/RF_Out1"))
 (segment (start 112.5 94) (end 111.634214 94) (width 1) (layer "F.Cu") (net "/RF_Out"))
 (segment (start 108.825 92.046386) (end 108.825 90.5) (width 1) (layer "F.Cu") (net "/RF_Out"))
 (arc (start 111.634214 94) (mid 110.32765 93.740109) (end 109.22 93) (width 1) (layer "F.Cu") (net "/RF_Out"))
 (arc (start 109.22 93) (mid 108.927657 92.562478) (end 108.825 92.046386) (width 1) (layer "F.Cu") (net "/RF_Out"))
 (segment (start 102.572893 92.5) (end 101.5 92.5) (width 1) (layer "F.Cu") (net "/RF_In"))
 (arc (start 103.78 93) (mid 103.226175 92.629946) (end 102.572893 92.5) (width 1) (layer "F.Cu") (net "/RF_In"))
 (segment (start 101.5 94.225) (end 102.475 94.225) (width 1) (layer "F.Cu") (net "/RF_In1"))
 (segment (start 102.475 94.225) (end 102.5 94.2) (width 1) (layer "F.Cu") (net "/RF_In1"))
 (segment (start 101.4875 96) (end 101.4875 94.255178) (width 1) (layer "F.Cu") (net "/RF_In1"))
 (via (at 102.5 94.2) (size 0.8) (drill 0.5) (layers "F.Cu" "B.Cu") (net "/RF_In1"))
 (arc (start 101.4875 94.255178) (mid 101.490748 94.238846) (end 101.5 94.225) (width 1) (layer "F.Cu") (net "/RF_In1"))
 (segment (start 102.5 94.2) (end 101.986136 93.686136) (width 1) (layer "B.Cu") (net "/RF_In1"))
 (arc (start 101.986136 93.686136) (mid 101.626342 93.147668) (end 101.5 92.5125) (width 1) (layer "B.Cu") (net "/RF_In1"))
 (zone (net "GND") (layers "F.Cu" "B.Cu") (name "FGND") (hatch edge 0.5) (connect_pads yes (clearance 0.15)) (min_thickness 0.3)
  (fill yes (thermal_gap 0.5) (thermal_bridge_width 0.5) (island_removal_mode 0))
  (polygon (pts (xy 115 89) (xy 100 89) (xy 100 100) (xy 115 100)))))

